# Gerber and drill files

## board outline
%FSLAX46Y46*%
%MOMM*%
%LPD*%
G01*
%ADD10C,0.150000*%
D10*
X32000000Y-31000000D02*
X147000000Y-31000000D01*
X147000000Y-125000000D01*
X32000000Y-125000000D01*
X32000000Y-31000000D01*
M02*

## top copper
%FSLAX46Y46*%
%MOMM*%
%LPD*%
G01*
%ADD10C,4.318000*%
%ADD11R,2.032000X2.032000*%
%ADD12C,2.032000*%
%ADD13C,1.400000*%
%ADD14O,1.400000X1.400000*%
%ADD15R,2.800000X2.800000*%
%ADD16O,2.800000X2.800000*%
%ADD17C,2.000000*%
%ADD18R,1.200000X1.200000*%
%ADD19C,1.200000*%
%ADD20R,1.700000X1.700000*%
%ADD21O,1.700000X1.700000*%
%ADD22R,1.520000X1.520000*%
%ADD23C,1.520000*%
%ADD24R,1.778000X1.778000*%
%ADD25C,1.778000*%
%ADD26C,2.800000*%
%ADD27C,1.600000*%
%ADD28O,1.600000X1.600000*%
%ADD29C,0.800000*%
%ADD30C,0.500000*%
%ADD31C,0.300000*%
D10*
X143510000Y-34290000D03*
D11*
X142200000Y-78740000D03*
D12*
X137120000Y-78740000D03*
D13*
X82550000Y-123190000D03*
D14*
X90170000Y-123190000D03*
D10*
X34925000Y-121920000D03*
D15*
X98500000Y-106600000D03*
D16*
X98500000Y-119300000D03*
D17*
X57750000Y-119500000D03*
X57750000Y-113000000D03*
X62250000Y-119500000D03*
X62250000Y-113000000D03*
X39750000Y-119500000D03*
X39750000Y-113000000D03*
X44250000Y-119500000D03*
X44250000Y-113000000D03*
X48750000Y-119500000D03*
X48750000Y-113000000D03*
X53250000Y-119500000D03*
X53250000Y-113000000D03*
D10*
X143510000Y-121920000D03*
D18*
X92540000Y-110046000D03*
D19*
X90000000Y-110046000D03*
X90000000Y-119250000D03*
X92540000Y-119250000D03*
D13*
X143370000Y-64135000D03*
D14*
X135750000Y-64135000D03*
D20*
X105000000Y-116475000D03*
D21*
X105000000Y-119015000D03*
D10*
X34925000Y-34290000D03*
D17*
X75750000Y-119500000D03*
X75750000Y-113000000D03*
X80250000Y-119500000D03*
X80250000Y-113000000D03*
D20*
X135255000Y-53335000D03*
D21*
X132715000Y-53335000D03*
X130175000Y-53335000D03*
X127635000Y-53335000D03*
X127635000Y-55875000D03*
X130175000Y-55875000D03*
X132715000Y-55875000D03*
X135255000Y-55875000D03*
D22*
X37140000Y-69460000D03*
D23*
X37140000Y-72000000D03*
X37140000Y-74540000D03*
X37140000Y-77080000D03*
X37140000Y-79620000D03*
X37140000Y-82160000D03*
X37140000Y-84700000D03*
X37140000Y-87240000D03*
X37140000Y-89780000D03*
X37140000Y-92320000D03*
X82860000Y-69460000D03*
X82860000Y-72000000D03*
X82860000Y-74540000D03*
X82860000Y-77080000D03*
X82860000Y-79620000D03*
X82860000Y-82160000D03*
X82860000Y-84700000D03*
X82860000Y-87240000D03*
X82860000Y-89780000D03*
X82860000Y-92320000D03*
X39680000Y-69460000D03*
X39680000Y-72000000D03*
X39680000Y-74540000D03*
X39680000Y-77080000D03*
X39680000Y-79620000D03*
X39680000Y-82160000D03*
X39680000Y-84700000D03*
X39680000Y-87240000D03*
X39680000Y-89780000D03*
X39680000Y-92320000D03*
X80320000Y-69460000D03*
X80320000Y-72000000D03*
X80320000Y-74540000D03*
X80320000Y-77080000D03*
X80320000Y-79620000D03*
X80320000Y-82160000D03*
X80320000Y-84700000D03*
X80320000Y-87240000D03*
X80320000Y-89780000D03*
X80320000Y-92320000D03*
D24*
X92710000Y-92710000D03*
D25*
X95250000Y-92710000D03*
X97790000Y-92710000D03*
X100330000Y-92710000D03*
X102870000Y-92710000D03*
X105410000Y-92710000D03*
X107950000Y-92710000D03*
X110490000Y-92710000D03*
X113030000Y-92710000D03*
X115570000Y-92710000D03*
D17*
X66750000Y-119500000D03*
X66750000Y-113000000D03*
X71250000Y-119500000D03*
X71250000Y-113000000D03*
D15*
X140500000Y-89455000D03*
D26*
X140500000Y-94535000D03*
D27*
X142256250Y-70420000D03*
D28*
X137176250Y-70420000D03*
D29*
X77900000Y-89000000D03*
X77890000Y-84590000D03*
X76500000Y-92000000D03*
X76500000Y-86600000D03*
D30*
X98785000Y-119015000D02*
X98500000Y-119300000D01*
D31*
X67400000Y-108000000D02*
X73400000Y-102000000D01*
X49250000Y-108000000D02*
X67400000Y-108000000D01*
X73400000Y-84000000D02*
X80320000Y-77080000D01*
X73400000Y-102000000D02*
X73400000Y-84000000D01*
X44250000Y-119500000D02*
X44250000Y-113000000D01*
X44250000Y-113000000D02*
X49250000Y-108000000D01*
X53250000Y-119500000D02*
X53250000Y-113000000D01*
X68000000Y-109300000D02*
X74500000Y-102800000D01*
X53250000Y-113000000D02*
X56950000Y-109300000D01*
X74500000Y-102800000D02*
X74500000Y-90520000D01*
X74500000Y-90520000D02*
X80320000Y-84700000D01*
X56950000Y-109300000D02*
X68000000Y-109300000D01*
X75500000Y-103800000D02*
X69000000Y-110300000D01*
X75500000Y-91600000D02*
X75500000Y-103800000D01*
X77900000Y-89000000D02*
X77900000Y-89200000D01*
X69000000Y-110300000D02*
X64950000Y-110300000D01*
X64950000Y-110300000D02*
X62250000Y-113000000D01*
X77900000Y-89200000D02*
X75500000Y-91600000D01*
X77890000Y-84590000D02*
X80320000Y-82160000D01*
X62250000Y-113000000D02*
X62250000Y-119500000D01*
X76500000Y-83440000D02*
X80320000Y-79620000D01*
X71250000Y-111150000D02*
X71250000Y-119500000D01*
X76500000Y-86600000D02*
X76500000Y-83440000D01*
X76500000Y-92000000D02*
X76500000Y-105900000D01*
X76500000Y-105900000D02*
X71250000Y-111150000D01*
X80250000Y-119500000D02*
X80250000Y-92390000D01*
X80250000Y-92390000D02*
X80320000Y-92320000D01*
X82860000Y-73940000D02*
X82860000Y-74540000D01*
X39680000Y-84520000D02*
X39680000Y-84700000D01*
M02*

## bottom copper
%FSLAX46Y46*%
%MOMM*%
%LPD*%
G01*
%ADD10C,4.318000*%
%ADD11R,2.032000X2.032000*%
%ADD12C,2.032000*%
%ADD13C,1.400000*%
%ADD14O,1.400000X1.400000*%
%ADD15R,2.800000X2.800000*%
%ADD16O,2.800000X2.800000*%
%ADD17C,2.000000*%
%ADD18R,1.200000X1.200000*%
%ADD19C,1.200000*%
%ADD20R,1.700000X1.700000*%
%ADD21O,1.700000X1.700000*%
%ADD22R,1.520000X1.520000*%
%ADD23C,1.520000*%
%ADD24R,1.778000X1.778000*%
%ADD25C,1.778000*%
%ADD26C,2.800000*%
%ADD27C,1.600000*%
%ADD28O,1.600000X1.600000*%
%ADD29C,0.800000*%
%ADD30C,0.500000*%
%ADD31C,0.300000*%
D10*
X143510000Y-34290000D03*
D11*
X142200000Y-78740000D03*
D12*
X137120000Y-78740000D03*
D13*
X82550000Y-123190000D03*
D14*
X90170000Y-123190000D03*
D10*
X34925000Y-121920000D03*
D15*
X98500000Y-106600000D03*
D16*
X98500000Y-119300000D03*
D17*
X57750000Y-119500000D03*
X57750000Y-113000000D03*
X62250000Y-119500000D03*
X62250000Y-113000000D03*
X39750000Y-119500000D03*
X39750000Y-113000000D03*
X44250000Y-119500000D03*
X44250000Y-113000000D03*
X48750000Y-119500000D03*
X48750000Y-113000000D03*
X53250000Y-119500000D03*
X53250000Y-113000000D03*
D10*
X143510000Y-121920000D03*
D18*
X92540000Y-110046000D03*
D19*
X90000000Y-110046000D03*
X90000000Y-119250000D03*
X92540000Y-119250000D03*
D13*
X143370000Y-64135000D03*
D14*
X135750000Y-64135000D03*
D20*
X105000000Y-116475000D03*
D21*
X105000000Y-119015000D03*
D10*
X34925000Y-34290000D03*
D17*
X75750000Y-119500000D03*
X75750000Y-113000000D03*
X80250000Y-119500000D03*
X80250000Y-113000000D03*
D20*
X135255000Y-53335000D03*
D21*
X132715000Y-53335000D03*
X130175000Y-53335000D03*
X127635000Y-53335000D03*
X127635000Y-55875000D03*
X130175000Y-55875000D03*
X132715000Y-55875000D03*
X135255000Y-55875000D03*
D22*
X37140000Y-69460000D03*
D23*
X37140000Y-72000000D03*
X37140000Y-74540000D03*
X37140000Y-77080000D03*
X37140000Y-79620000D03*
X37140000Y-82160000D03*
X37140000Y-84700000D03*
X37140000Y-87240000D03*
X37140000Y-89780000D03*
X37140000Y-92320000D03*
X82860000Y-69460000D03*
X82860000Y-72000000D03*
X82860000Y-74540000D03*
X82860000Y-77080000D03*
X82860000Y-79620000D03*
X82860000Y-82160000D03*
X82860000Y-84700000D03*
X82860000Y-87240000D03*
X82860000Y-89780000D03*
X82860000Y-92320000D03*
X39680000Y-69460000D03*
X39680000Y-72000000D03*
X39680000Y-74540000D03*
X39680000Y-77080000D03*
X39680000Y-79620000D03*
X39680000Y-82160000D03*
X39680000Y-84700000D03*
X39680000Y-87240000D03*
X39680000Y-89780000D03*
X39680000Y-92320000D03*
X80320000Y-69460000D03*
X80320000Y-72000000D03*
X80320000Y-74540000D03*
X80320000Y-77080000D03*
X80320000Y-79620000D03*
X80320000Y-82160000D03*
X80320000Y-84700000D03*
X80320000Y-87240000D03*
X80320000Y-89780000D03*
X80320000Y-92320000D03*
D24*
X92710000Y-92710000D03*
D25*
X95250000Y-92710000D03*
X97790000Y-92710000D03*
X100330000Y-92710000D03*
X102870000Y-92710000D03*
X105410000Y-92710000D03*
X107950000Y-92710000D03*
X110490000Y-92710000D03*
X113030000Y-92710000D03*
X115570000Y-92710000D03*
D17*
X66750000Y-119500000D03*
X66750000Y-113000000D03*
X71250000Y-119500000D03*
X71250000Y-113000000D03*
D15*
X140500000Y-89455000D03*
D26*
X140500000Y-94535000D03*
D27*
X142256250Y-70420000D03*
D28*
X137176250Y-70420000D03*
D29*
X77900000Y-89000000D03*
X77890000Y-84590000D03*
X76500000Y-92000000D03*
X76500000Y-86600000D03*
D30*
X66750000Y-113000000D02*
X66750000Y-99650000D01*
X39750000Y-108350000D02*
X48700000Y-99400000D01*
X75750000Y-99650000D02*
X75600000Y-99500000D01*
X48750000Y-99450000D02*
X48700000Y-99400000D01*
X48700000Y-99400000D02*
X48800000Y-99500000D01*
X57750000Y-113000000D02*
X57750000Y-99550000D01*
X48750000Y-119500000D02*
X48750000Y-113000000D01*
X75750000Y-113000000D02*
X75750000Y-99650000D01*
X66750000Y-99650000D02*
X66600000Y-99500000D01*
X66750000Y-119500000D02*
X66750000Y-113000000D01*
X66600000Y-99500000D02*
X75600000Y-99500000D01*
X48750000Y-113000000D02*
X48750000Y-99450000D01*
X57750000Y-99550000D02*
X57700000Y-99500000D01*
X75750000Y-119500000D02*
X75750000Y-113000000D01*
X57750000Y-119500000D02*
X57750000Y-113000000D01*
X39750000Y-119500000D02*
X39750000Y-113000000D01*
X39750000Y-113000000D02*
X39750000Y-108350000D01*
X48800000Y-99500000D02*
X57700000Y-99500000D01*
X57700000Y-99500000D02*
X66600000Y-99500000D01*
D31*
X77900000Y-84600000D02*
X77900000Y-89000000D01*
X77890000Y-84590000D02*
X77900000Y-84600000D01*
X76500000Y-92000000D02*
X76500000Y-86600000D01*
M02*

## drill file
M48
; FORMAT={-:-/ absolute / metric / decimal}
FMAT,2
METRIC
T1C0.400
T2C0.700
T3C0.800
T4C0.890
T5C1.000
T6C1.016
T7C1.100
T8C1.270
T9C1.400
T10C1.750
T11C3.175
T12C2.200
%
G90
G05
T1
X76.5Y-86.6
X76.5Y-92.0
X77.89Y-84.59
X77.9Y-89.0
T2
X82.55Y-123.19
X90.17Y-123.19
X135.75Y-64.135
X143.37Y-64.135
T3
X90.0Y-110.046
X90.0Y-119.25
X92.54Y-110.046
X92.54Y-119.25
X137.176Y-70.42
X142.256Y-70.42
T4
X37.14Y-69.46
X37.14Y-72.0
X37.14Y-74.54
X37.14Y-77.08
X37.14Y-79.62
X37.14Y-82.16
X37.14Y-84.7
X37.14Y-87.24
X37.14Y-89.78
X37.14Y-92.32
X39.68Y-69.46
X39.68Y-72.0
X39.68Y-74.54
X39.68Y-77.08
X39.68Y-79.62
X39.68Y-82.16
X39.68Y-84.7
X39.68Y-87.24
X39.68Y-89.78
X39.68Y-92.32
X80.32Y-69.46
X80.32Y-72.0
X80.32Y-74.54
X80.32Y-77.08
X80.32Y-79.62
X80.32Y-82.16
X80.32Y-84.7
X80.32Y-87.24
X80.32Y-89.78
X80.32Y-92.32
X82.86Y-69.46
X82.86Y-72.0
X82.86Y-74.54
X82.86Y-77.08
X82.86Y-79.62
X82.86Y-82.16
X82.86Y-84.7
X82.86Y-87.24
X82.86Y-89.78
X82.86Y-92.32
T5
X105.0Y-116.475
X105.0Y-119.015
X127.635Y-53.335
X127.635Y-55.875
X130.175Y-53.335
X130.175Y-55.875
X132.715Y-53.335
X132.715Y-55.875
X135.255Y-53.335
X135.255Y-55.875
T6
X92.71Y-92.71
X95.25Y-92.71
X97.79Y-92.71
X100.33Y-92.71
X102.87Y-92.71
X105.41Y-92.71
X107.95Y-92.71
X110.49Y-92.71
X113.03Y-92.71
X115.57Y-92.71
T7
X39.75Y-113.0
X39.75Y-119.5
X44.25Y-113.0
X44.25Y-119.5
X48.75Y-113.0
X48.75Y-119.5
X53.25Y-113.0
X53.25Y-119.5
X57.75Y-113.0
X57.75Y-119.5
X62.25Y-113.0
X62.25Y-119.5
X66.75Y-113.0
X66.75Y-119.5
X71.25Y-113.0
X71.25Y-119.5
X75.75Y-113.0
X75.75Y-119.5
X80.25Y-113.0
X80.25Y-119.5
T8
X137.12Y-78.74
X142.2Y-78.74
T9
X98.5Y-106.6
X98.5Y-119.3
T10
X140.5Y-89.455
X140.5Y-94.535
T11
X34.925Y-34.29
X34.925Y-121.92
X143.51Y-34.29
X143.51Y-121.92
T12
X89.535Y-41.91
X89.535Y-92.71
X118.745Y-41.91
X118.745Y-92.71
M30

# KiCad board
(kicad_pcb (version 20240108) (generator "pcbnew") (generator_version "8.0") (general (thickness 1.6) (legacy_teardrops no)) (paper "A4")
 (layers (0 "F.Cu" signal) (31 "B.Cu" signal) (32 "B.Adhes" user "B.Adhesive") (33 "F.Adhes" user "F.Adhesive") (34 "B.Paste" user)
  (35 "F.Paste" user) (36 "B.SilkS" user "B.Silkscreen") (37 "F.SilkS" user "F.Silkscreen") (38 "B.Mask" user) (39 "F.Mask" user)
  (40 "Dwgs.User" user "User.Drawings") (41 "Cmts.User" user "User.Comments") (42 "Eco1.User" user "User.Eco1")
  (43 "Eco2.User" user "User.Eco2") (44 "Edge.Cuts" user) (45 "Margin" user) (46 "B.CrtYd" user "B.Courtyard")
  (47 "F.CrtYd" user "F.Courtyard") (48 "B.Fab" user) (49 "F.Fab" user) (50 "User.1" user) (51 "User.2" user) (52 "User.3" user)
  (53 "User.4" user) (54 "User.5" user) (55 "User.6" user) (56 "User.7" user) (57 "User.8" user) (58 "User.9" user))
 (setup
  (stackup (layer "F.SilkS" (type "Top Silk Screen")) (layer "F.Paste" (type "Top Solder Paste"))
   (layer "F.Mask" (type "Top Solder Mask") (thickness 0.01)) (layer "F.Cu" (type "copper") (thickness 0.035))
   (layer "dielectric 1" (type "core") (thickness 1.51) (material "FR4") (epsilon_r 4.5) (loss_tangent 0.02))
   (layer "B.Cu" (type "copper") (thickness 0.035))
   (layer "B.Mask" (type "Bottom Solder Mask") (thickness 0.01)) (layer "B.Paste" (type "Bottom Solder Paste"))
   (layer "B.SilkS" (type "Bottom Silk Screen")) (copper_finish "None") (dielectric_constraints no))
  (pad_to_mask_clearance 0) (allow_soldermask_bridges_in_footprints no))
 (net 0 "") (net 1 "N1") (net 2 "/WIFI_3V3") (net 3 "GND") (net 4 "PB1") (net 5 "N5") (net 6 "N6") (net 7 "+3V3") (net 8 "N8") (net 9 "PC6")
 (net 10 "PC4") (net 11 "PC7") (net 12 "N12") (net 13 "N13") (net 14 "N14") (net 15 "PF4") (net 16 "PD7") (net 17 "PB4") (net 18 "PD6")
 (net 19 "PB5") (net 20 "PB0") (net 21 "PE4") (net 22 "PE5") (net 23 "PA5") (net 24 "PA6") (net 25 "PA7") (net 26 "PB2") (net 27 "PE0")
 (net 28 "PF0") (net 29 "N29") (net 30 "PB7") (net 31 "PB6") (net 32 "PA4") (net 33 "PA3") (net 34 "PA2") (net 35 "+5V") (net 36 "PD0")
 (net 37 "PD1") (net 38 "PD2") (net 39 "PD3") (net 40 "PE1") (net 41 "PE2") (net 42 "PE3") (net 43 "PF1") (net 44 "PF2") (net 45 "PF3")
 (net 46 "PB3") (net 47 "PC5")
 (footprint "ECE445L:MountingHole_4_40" (layer "F.Cu") (at 143.51 34.29)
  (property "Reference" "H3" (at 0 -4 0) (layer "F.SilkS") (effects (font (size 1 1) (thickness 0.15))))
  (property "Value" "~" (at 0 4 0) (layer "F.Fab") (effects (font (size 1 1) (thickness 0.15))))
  (pad "1" thru_hole circle (at 0 0) (size 4.318 4.318) (drill 3.175) (layers "*.Cu" "*.Mask") (remove_unused_layers no) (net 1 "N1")))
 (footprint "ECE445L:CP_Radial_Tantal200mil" (layer "F.Cu") (at 142.2 78.74 180)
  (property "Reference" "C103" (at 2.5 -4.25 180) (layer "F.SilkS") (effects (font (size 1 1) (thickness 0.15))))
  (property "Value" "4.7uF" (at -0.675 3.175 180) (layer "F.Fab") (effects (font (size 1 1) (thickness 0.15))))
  (pad "1" thru_hole rect (at 0 0 180) (size 2.032 2.032) (drill 1.27) (layers "*.Cu" "*.Mask") (remove_unused_layers no)
   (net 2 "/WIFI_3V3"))
  (pad "2" thru_hole circle (at 5.08 0 180) (size 2.032 2.032) (drill 1.27) (layers "*.Cu" "*.Mask") (remove_unused_layers no) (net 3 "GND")))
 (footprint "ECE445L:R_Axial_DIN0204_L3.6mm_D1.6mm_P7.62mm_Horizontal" (layer "F.Cu") (at 82.55 123.19)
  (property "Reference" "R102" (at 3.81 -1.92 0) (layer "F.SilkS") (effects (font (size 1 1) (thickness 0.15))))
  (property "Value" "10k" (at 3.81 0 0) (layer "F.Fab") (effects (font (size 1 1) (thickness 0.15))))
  (pad "1" thru_hole circle (at 0 0) (size 1.4 1.4) (drill 0.7) (layers "*.Cu" "*.Mask") (remove_unused_layers no) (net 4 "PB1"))
  (pad "2" thru_hole oval (at 7.62 0) (size 1.4 1.4) (drill 0.7) (layers "*.Cu" "*.Mask") (remove_unused_layers no) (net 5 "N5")))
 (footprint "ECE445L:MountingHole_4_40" (layer "F.Cu") (at 34.925 121.92)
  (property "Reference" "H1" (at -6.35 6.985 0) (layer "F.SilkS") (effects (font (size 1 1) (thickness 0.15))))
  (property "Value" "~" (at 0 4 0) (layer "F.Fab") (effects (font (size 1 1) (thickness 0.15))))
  (pad "1" thru_hole circle (at 0 0) (size 4.318 4.318) (drill 3.175) (layers "*.Cu" "*.Mask") (remove_unused_layers no) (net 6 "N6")))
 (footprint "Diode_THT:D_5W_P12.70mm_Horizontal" (layer "F.Cu") (at 98.5 106.6 -90)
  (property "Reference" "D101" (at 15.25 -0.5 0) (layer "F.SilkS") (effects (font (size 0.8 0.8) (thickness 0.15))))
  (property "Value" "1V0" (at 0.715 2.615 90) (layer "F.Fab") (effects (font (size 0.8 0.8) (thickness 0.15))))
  (pad "1" thru_hole rect (at 0 0 270) (size 2.8 2.8) (drill 1.4) (layers "*.Cu" "*.Mask") (remove_unused_layers no) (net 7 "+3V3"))
  (pad "2" thru_hole oval (at 12.7 0 270) (size 2.8 2.8) (drill 1.4) (layers "*.Cu" "*.Mask") (remove_unused_layers no) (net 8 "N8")))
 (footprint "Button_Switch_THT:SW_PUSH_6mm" (layer "F.Cu") (at 57.75 119.5 90)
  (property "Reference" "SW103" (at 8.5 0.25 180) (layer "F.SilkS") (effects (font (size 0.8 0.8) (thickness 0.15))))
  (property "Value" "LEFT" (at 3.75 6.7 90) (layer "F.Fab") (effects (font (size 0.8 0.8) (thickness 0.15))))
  (pad "1" thru_hole circle (at 0 0 180) (size 2 2) (drill 1.1) (layers "*.Cu" "*.Mask") (remove_unused_layers no) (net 3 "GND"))
  (pad "1" thru_hole circle (at 6.5 0 180) (size 2 2) (drill 1.1) (layers "*.Cu" "*.Mask") (remove_unused_layers no) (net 3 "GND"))
  (pad "2" thru_hole circle (at 0 4.5 180) (size 2 2) (drill 1.1) (layers "*.Cu" "*.Mask") (remove_unused_layers no) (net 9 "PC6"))
  (pad "2" thru_hole circle (at 6.5 4.5 180) (size 2 2) (drill 1.1) (layers "*.Cu" "*.Mask") (remove_unused_layers no) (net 9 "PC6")))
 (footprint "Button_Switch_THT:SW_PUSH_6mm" (layer "F.Cu") (at 39.75 119.5 90)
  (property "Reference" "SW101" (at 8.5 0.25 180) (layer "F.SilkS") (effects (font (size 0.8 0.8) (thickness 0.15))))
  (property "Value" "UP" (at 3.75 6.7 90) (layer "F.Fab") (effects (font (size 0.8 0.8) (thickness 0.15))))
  (pad "1" thru_hole circle (at 0 0 180) (size 2 2) (drill 1.1) (layers "*.Cu" "*.Mask") (remove_unused_layers no) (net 3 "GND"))
  (pad "1" thru_hole circle (at 6.5 0 180) (size 2 2) (drill 1.1) (layers "*.Cu" "*.Mask") (remove_unused_layers no) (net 3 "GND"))
  (pad "2" thru_hole circle (at 0 4.5 180) (size 2 2) (drill 1.1) (layers "*.Cu" "*.Mask") (remove_unused_layers no) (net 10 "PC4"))
  (pad "2" thru_hole circle (at 6.5 4.5 180) (size 2 2) (drill 1.1) (layers "*.Cu" "*.Mask") (remove_unused_layers no) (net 10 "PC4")))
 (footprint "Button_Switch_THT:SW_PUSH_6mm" (layer "F.Cu") (at 48.75 119.5 90)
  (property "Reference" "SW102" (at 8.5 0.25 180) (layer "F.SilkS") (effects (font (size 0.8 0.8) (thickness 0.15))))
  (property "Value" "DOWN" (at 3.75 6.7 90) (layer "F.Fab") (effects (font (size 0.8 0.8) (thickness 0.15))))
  (pad "1" thru_hole circle (at 0 0 180) (size 2 2) (drill 1.1) (layers "*.Cu" "*.Mask") (remove_unused_layers no) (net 3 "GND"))
  (pad "1" thru_hole circle (at 6.5 0 180) (size 2 2) (drill 1.1) (layers "*.Cu" "*.Mask") (remove_unused_layers no) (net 3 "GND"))
  (pad "2" thru_hole circle (at 0 4.5 180) (size 2 2) (drill 1.1) (layers "*.Cu" "*.Mask") (remove_unused_layers no) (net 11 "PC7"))
  (pad "2" thru_hole circle (at 6.5 4.5 180) (size 2 2) (drill 1.1) (layers "*.Cu" "*.Mask") (remove_unused_layers no) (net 11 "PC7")))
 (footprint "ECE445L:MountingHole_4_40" (layer "F.Cu") (at 143.51 121.92)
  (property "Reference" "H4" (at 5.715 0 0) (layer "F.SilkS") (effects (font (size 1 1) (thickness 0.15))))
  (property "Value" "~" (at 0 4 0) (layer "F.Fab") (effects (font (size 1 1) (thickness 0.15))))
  (pad "1" thru_hole circle (at 0 0) (size 4.318 4.318) (drill 3.175) (layers "*.Cu" "*.Mask") (remove_unused_layers no) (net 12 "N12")))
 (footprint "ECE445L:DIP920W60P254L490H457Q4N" (layer "F.Cu") (at 91.27 114.648 -90)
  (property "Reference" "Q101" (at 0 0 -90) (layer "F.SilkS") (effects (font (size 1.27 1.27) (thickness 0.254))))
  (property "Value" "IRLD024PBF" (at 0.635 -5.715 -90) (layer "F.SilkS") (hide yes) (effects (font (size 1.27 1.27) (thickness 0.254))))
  (pad "1" thru_hole rect (at -4.602 -1.27 270) (size 1.2 1.2) (drill 0.8) (layers "*.Cu" "*.Mask") (remove_unused_layers no) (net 8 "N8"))
  (pad "2" thru_hole circle (at -4.602 1.27 270) (size 1.2 1.2) (drill 0.8) (layers "*.Cu" "*.Mask") (remove_unused_layers no) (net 8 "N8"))
  (pad "3" thru_hole circle (at 4.602 1.27 270) (size 1.2 1.2) (drill 0.8) (layers "*.Cu" "*.Mask") (remove_unused_layers no) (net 5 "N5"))
  (pad "4" thru_hole circle (at 4.602 -1.27 270) (size 1.2 1.2) (drill 0.8) (layers "*.Cu" "*.Mask") (remove_unused_layers no) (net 3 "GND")))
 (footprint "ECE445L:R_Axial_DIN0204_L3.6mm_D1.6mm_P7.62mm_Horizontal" (layer "F.Cu") (at 143.37 64.135 180)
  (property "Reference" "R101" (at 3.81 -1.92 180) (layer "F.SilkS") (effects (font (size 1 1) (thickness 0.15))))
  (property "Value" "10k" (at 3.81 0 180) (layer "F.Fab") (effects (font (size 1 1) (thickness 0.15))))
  (pad "1" thru_hole circle (at 0 0 180) (size 1.4 1.4) (drill 0.7) (layers "*.Cu" "*.Mask") (remove_unused_layers no) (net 2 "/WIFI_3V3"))
  (pad "2" thru_hole oval (at 7.62 0 180) (size 1.4 1.4) (drill 0.7) (layers "*.Cu" "*.Mask") (remove_unused_layers no) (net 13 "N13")))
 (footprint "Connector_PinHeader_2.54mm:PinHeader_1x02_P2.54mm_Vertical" (layer "F.Cu") (at 105 116.475)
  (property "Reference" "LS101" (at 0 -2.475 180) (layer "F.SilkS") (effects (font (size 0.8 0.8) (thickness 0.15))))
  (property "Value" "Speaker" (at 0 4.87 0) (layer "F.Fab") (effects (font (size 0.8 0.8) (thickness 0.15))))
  (pad "1" thru_hole rect (at 0 0) (size 1.7 1.7) (drill 1) (layers "*.Cu" "*.Mask") (remove_unused_layers no) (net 7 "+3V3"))
  (pad "2" thru_hole oval (at 0 2.54) (size 1.7 1.7) (drill 1) (layers "*.Cu" "*.Mask") (remove_unused_layers no) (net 8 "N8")))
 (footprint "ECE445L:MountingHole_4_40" (layer "F.Cu") (at 34.925 34.29)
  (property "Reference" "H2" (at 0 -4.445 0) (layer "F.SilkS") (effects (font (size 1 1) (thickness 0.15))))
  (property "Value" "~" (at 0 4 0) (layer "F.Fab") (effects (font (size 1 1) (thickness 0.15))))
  (pad "1" thru_hole circle (at 0 0) (size 4.318 4.318) (drill 3.175) (layers "*.Cu" "*.Mask") (remove_unused_layers no) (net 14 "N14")))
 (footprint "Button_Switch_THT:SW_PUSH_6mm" (layer "F.Cu") (at 75.75 119.5 90)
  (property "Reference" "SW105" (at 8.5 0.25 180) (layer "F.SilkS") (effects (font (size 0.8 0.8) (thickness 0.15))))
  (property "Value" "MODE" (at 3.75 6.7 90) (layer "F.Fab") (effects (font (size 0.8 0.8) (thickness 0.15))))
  (pad "1" thru_hole circle (at 0 0 180) (size 2 2) (drill 1.1) (layers "*.Cu" "*.Mask") (remove_unused_layers no) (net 3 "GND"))
  (pad "1" thru_hole circle (at 6.5 0 180) (size 2 2) (drill 1.1) (layers "*.Cu" "*.Mask") (remove_unused_layers no) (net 3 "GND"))
  (pad "2" thru_hole circle (at 0 4.5 180) (size 2 2) (drill 1.1) (layers "*.Cu" "*.Mask") (remove_unused_layers no) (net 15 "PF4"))
  (pad "2" thru_hole circle (at 6.5 4.5 180) (size 2 2) (drill 1.1) (layers "*.Cu" "*.Mask") (remove_unused_layers no) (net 15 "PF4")))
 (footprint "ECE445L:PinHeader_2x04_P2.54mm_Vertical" (layer "F.Cu") (at 135.255 53.335 -90)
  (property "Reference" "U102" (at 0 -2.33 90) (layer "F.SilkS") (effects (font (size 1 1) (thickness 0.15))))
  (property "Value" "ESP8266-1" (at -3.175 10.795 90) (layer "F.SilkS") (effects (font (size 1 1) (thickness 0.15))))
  (pad "1" thru_hole rect (at 0 0 270) (size 1.7 1.7) (drill 1) (layers "*.Cu" "*.Mask") (remove_unused_layers no) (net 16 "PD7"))
  (pad "2" thru_hole oval (at 0 2.54 270) (size 1.7 1.7) (drill 1) (layers "*.Cu" "*.Mask") (remove_unused_layers no) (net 2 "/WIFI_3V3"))
  (pad "3" thru_hole oval (at 0 5.08 270) (size 1.7 1.7) (drill 1) (layers "*.Cu" "*.Mask") (remove_unused_layers no) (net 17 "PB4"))
  (pad "4" thru_hole oval (at 0 7.62 270) (size 1.7 1.7) (drill 1) (layers "*.Cu" "*.Mask") (remove_unused_layers no) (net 3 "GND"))
  (pad "5" thru_hole oval (at 2.54 7.62 270) (size 1.7 1.7) (drill 1) (layers "*.Cu" "*.Mask") (remove_unused_layers no) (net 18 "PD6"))
  (pad "6" thru_hole oval (at 2.54 5.08 270) (size 1.7 1.7) (drill 1) (layers "*.Cu" "*.Mask") (remove_unused_layers no) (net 13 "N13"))
  (pad "7" thru_hole oval (at 2.54 2.54 270) (size 1.7 1.7) (drill 1) (layers "*.Cu" "*.Mask") (remove_unused_layers no) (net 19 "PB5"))
  (pad "8" thru_hole oval (at 2.54 0 270) (size 1.7 1.7) (drill 1) (layers "*.Cu" "*.Mask") (remove_unused_layers no) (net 2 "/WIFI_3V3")))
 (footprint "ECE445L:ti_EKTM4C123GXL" (layer "F.Cu") (at 60 72)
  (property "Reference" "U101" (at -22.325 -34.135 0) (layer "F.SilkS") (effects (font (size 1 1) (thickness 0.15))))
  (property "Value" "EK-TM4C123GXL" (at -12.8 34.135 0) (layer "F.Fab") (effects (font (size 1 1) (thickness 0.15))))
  (pad "J1_1" thru_hole rect (at -22.86 -2.54) (size 1.52 1.52) (drill 0.89) (layers "*.Cu" "*.Mask") (remove_unused_layers no)
   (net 7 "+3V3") (solder_mask_margin 0.102))
  (pad "J1_2" thru_hole circle (at -22.86 0) (size 1.52 1.52) (drill 0.89) (layers "*.Cu" "*.Mask") (remove_unused_layers no) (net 19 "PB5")
   (solder_mask_margin 0.102))
  (pad "J1_3" thru_hole circle (at -22.86 2.54) (size 1.52 1.52) (drill 0.89) (layers "*.Cu" "*.Mask") (remove_unused_layers no)
   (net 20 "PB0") (solder_mask_margin 0.102))
  (pad "J1_4" thru_hole circle (at -22.86 5.08) (size 1.52 1.52) (drill 0.89) (layers "*.Cu" "*.Mask") (remove_unused_layers no)
   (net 4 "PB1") (solder_mask_margin 0.102))
  (pad "J1_5" thru_hole circle (at -22.86 7.62) (size 1.52 1.52) (drill 0.89) (layers "*.Cu" "*.Mask") (remove_unused_layers no)
   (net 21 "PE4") (solder_mask_margin 0.102))
  (pad "J1_6" thru_hole circle (at -22.86 10.16) (size 1.52 1.52) (drill 0.89) (layers "*.Cu" "*.Mask") (remove_unused_layers no)
   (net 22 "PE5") (solder_mask_margin 0.102))
  (pad "J1_7" thru_hole circle (at -22.86 12.7) (size 1.52 1.52) (drill 0.89) (layers "*.Cu" "*.Mask") (remove_unused_layers no)
   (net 17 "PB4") (solder_mask_margin 0.102))
  (pad "J1_8" thru_hole circle (at -22.86 15.24) (size 1.52 1.52) (drill 0.89) (layers "*.Cu" "*.Mask") (remove_unused_layers no)
   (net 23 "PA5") (solder_mask_margin 0.102))
  (pad "J1_9" thru_hole circle (at -22.86 17.78) (size 1.52 1.52) (drill 0.89) (layers "*.Cu" "*.Mask") (remove_unused_layers no)
   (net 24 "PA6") (solder_mask_margin 0.102))
  (pad "J1_10" thru_hole circle (at -22.86 20.32) (size 1.52 1.52) (drill 0.89) (layers "*.Cu" "*.Mask") (remove_unused_layers no)
   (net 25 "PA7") (solder_mask_margin 0.102))
  (pad "J2_1" thru_hole circle (at 22.86 -2.54) (size 1.52 1.52) (drill 0.89) (layers "*.Cu" "*.Mask") (remove_unused_layers no)
   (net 3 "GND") (solder_mask_margin 0.102))
  (pad "J2_2" thru_hole circle (at 22.86 0) (size 1.52 1.52) (drill 0.89) (layers "*.Cu" "*.Mask") (remove_unused_layers no) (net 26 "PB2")
   (solder_mask_margin 0.102))
  (pad "J2_3" thru_hole circle (at 22.86 2.54) (size 1.52 1.52) (drill 0.89) (layers "*.Cu" "*.Mask") (remove_unused_layers no)
   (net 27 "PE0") (solder_mask_margin 0.102))
  (pad "J2_4" thru_hole circle (at 22.86 5.08) (size 1.52 1.52) (drill 0.89) (layers "*.Cu" "*.Mask") (remove_unused_layers no)
   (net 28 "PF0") (solder_mask_margin 0.102))
  (pad "J2_5" thru_hole circle (at 22.86 7.62) (size 1.52 1.52) (drill 0.89) (layers "*.Cu" "*.Mask") (remove_unused_layers no)
   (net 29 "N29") (solder_mask_margin 0.102))
  (pad "J2_6" thru_hole circle (at 22.86 10.16) (size 1.52 1.52) (drill 0.89) (layers "*.Cu" "*.Mask") (remove_unused_layers no)
   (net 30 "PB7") (solder_mask_margin 0.102))
  (pad "J2_7" thru_hole circle (at 22.86 12.7) (size 1.52 1.52) (drill 0.89) (layers "*.Cu" "*.Mask") (remove_unused_layers no)
   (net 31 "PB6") (solder_mask_margin 0.102))
  (pad "J2_8" thru_hole circle (at 22.86 15.24) (size 1.52 1.52) (drill 0.89) (layers "*.Cu" "*.Mask") (remove_unused_layers no)
   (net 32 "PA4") (solder_mask_margin 0.102))
  (pad "J2_9" thru_hole circle (at 22.86 17.78) (size 1.52 1.52) (drill 0.89) (layers "*.Cu" "*.Mask") (remove_unused_layers no)
   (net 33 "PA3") (solder_mask_margin 0.102))
  (pad "J2_10" thru_hole circle (at 22.86 20.32) (size 1.52 1.52) (drill 0.89) (layers "*.Cu" "*.Mask") (remove_unused_layers no)
   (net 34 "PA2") (solder_mask_margin 0.102))
  (pad "J3_1" thru_hole circle (at -20.32 -2.54) (size 1.52 1.52) (drill 0.89) (layers "*.Cu" "*.Mask") (remove_unused_layers no)
   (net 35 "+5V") (solder_mask_margin 0.102))
  (pad "J3_2" thru_hole circle (at -20.32 0) (size 1.52 1.52) (drill 0.89) (layers "*.Cu" "*.Mask") (remove_unused_layers no) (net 3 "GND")
   (solder_mask_margin 0.102))
  (pad "J3_3" thru_hole circle (at -20.32 2.54) (size 1.52 1.52) (drill 0.89) (layers "*.Cu" "*.Mask") (remove_unused_layers no)
   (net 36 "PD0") (solder_mask_margin 0.102))
  (pad "J3_4" thru_hole circle (at -20.32 5.08) (size 1.52 1.52) (drill 0.89) (layers "*.Cu" "*.Mask") (remove_unused_layers no)
   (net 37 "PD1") (solder_mask_margin 0.102))
  (pad "J3_5" thru_hole circle (at -20.32 7.62) (size 1.52 1.52) (drill 0.89) (layers "*.Cu" "*.Mask") (remove_unused_layers no)
   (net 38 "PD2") (solder_mask_margin 0.102))
  (pad "J3_6" thru_hole circle (at -20.32 10.16) (size 1.52 1.52) (drill 0.89) (layers "*.Cu" "*.Mask") (remove_unused_layers no)
   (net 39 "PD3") (solder_mask_margin 0.102))
  (pad "J3_7" thru_hole circle (at -20.32 12.7) (size 1.52 1.52) (drill 0.89) (layers "*.Cu" "*.Mask") (remove_unused_layers no)
   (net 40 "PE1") (solder_mask_margin 0.102))
  (pad "J3_8" thru_hole circle (at -20.32 15.24) (size 1.52 1.52) (drill 0.89) (layers "*.Cu" "*.Mask") (remove_unused_layers no)
   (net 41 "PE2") (solder_mask_margin 0.102))
  (pad "J3_9" thru_hole circle (at -20.32 17.78) (size 1.52 1.52) (drill 0.89) (layers "*.Cu" "*.Mask") (remove_unused_layers no)
   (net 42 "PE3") (solder_mask_margin 0.102))
  (pad "J3_10" thru_hole circle (at -20.32 20.32) (size 1.52 1.52) (drill 0.89) (layers "*.Cu" "*.Mask") (remove_unused_layers no)
   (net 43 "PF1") (solder_mask_margin 0.102))
  (pad "J4_1" thru_hole circle (at 20.32 -2.54) (size 1.52 1.52) (drill 0.89) (layers "*.Cu" "*.Mask") (remove_unused_layers no)
   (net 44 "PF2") (solder_mask_margin 0.102))
  (pad "J4_2" thru_hole circle (at 20.32 0) (size 1.52 1.52) (drill 0.89) (layers "*.Cu" "*.Mask") (remove_unused_layers no) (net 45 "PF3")
   (solder_mask_margin 0.102))
  (pad "J4_3" thru_hole circle (at 20.32 2.54) (size 1.52 1.52) (drill 0.89) (layers "*.Cu" "*.Mask") (remove_unused_layers no)
   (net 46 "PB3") (solder_mask_margin 0.102))
  (pad "J4_4" thru_hole circle (at 20.32 5.08) (size 1.52 1.52) (drill 0.89) (layers "*.Cu" "*.Mask") (remove_unused_layers no)
   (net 10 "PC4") (solder_mask_margin 0.102))
  (pad "J4_5" thru_hole circle (at 20.32 7.62) (size 1.52 1.52) (drill 0.89) (layers "*.Cu" "*.Mask") (remove_unused_layers no)
   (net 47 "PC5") (solder_mask_margin 0.102))
  (pad "J4_6" thru_hole circle (at 20.32 10.16) (size 1.52 1.52) (drill 0.89) (layers "*.Cu" "*.Mask") (remove_unused_layers no)
   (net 9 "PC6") (solder_mask_margin 0.102))
  (pad "J4_7" thru_hole circle (at 20.32 12.7) (size 1.52 1.52) (drill 0.89) (layers "*.Cu" "*.Mask") (remove_unused_layers no)
   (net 11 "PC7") (solder_mask_margin 0.102))
  (pad "J4_8" thru_hole circle (at 20.32 15.24) (size 1.52 1.52) (drill 0.89) (layers "*.Cu" "*.Mask") (remove_unused_layers no)
   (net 18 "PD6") (solder_mask_margin 0.102))
  (pad "J4_9" thru_hole circle (at 20.32 17.78) (size 1.52 1.52) (drill 0.89) (layers "*.Cu" "*.Mask") (remove_unused_layers no)
   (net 16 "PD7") (solder_mask_margin 0.102))
  (pad "J4_10" thru_hole circle (at 20.32 20.32) (size 1.52 1.52) (drill 0.89) (layers "*.Cu" "*.Mask") (remove_unused_layers no)
   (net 15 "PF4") (solder_mask_margin 0.102)))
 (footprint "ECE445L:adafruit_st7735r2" (layer "F.Cu") (at 104.14 67.31)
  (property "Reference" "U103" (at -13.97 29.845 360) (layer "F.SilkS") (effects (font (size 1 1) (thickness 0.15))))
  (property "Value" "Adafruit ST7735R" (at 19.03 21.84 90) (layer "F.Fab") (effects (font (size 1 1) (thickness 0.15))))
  (pad "" np_thru_hole circle (at -14.605 -25.4 90) (size 2.2 2.2) (drill 2.2) (layers "*.Cu" "*.Mask"))
  (pad "" np_thru_hole circle (at -14.605 25.4 90) (size 2.2 2.2) (drill 2.2) (layers "F&B.Cu" "*.Mask"))
  (pad "" np_thru_hole circle (at 14.605 -25.4 90) (size 2.2 2.2) (drill 2.2) (layers "F&B.Cu" "*.Mask"))
  (pad "" np_thru_hole circle (at 14.605 25.4 90) (size 2.2 2.2) (drill 2.2) (layers "F&B.Cu" "*.Mask"))
  (pad "1" thru_hole rect (at -11.43 25.4 90) (size 1.778 1.778) (drill 1.016) (layers "*.Cu" "*.Mask") (remove_unused_layers no)
   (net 3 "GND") (solder_mask_margin 0.102))
  (pad "2" thru_hole circle (at -8.89 25.4 90) (size 1.778 1.778) (drill 1.016) (layers "*.Cu" "*.Mask") (remove_unused_layers no)
   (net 7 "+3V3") (solder_mask_margin 0.102))
  (pad "3" thru_hole circle (at -6.35 25.4 90) (size 1.778 1.778) (drill 1.016) (layers "*.Cu" "*.Mask") (remove_unused_layers no)
   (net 25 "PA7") (solder_mask_margin 0.102))
  (pad "4" thru_hole circle (at -3.81 25.4 90) (size 1.778 1.778) (drill 1.016) (layers "*.Cu" "*.Mask") (remove_unused_layers no)
   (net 24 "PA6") (solder_mask_margin 0.102))
  (pad "5" thru_hole circle (at -1.27 25.4 90) (size 1.778 1.778) (drill 1.016) (layers "*.Cu" "*.Mask") (remove_unused_layers no)
   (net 20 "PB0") (solder_mask_margin 0.102))
  (pad "6" thru_hole circle (at 1.27 25.4 90) (size 1.778 1.778) (drill 1.016) (layers "*.Cu" "*.Mask") (remove_unused_layers no)
   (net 33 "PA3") (solder_mask_margin 0.102))
  (pad "7" thru_hole circle (at 3.81 25.4 90) (size 1.778 1.778) (drill 1.016) (layers "*.Cu" "*.Mask") (remove_unused_layers no)
   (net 23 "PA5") (solder_mask_margin 0.102))
  (pad "8" thru_hole circle (at 6.35 25.4 90) (size 1.778 1.778) (drill 1.016) (layers "*.Cu" "*.Mask") (remove_unused_layers no)
   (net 34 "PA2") (solder_mask_margin 0.102))
  (pad "9" thru_hole circle (at 8.89 25.4 90) (size 1.778 1.778) (drill 1.016) (layers "*.Cu" "*.Mask") (remove_unused_layers no)
   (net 32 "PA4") (solder_mask_margin 0.102))
  (pad "10" thru_hole circle (at 11.43 25.4 90) (size 1.778 1.778) (drill 1.016) (layers "*.Cu" "*.Mask") (remove_unused_layers no)
   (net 7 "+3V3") (solder_mask_margin 0.102)))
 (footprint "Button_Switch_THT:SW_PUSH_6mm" (layer "F.Cu") (at 66.75 119.5 90)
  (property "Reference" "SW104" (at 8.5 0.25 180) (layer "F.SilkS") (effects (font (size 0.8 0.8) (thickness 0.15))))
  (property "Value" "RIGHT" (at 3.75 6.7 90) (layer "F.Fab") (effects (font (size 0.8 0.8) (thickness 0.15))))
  (pad "1" thru_hole circle (at 0 0 180) (size 2 2) (drill 1.1) (layers "*.Cu" "*.Mask") (remove_unused_layers no) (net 3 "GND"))
  (pad "1" thru_hole circle (at 6.5 0 180) (size 2 2) (drill 1.1) (layers "*.Cu" "*.Mask") (remove_unused_layers no) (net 3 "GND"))
  (pad "2" thru_hole circle (at 0 4.5 180) (size 2 2) (drill 1.1) (layers "*.Cu" "*.Mask") (remove_unused_layers no) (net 47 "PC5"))
  (pad "2" thru_hole circle (at 6.5 4.5 180) (size 2 2) (drill 1.1) (layers "*.Cu" "*.Mask") (remove_unused_layers no) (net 47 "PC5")))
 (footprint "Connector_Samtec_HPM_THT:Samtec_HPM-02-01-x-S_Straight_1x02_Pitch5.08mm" (layer "F.Cu") (at 140.5 89.455)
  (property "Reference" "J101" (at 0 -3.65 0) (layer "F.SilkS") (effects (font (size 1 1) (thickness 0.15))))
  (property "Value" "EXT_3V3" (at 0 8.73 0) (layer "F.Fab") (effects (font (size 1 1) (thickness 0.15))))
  (pad "1" thru_hole rect (at 0 0) (size 2.8 2.8) (drill 1.75) (layers "*.Cu" "*.Mask") (remove_unused_layers no) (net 2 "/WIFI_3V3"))
  (pad "2" thru_hole circle (at 0 5.08) (size 2.8 2.8) (drill 1.75) (layers "*.Cu" "*.Mask") (remove_unused_layers no) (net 3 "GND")))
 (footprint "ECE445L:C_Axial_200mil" (layer "F.Cu") (at 142.25625 70.42 180)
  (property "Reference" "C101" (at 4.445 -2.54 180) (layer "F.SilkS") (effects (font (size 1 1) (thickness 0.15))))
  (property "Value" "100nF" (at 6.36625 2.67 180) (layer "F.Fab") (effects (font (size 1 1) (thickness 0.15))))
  (pad "1" thru_hole circle (at 0 0 180) (size 1.6 1.6) (drill 0.8) (layers "*.Cu" "*.Mask") (remove_unused_layers no) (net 2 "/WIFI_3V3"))
  (pad "2" thru_hole oval (at 5.08 0 180) (size 1.6 1.6) (drill 0.8) (layers "*.Cu" "*.Mask") (remove_unused_layers no) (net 3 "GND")))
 (gr_rect (start 32 31) (end 147 125) (stroke (width 0.15) (type default)) (fill none) (layer "Edge.Cuts"))
 (segment (start 66.75 113) (end 66.75 99.65) (width 0.5) (layer "B.Cu") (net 3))
 (segment (start 39.75 108.35) (end 48.7 99.4) (width 0.5) (layer "B.Cu") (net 3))
 (segment (start 75.75 99.65) (end 75.6 99.5) (width 0.5) (layer "B.Cu") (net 3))
 (segment (start 48.75 99.45) (end 48.7 99.4) (width 0.5) (layer "B.Cu") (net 3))
 (segment (start 48.7 99.4) (end 48.8 99.5) (width 0.5) (layer "B.Cu") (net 3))
 (segment (start 57.75 113) (end 57.75 99.55) (width 0.5) (layer "B.Cu") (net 3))
 (segment (start 48.75 119.5) (end 48.75 113) (width 0.5) (layer "B.Cu") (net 3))
 (segment (start 75.75 113) (end 75.75 99.65) (width 0.5) (layer "B.Cu") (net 3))
 (segment (start 66.75 99.65) (end 66.6 99.5) (width 0.5) (layer "B.Cu") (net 3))
 (segment (start 66.75 119.5) (end 66.75 113) (width 0.5) (layer "B.Cu") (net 3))
 (segment (start 66.6 99.5) (end 75.6 99.5) (width 0.5) (layer "B.Cu") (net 3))
 (segment (start 48.75 113) (end 48.75 99.45) (width 0.5) (layer "B.Cu") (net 3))
 (segment (start 57.75 99.55) (end 57.7 99.5) (width 0.5) (layer "B.Cu") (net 3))
 (segment (start 75.75 119.5) (end 75.75 113) (width 0.5) (layer "B.Cu") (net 3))
 (segment (start 57.75 119.5) (end 57.75 113) (width 0.5) (layer "B.Cu") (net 3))
 (segment (start 39.75 119.5) (end 39.75 113) (width 0.5) (layer "B.Cu") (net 3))
 (segment (start 39.75 113) (end 39.75 108.35) (width 0.5) (layer "B.Cu") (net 3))
 (segment (start 48.8 99.5) (end 57.7 99.5) (width 0.5) (layer "B.Cu") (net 3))
 (segment (start 57.7 99.5) (end 66.6 99.5) (width 0.5) (layer "B.Cu") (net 3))
 (segment (start 98.785 119.015) (end 98.5 119.3) (width 0.5) (layer "F.Cu") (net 8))
 (segment (start 67.4 108) (end 73.4 102) (width 0.3) (layer "F.Cu") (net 10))
 (segment (start 49.25 108) (end 67.4 108) (width 0.3) (layer "F.Cu") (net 10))
 (segment (start 73.4 84) (end 80.32 77.08) (width 0.3) (layer "F.Cu") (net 10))
 (segment (start 73.4 102) (end 73.4 84) (width 0.3) (layer "F.Cu") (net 10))
 (segment (start 44.25 119.5) (end 44.25 113) (width 0.3) (layer "F.Cu") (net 10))
 (segment (start 44.25 113) (end 49.25 108) (width 0.3) (layer "F.Cu") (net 10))
 (segment (start 53.25 119.5) (end 53.25 113) (width 0.3) (layer "F.Cu") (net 11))
 (segment (start 68 109.3) (end 74.5 102.8) (width 0.3) (layer "F.Cu") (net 11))
 (segment (start 53.25 113) (end 56.95 109.3) (width 0.3) (layer "F.Cu") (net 11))
 (segment (start 74.5 102.8) (end 74.5 90.52) (width 0.3) (layer "F.Cu") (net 11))
 (segment (start 74.5 90.52) (end 80.32 84.7) (width 0.3) (layer "F.Cu") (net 11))
 (segment (start 56.95 109.3) (end 68 109.3) (width 0.3) (layer "F.Cu") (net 11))
 (segment (start 75.5 103.8) (end 69 110.3) (width 0.3) (layer "F.Cu") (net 9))
 (segment (start 75.5 91.6) (end 75.5 103.8) (width 0.3) (layer "F.Cu") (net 9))
 (segment (start 77.9 89) (end 77.9 89.2) (width 0.3) (layer "F.Cu") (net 9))
 (segment (start 69 110.3) (end 64.95 110.3) (width 0.3) (layer "F.Cu") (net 9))
 (segment (start 64.95 110.3) (end 62.25 113) (width 0.3) (layer "F.Cu") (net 9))
 (segment (start 77.9 89.2) (end 75.5 91.6) (width 0.3) (layer "F.Cu") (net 9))
 (segment (start 77.89 84.59) (end 80.32 82.16) (width 0.3) (layer "F.Cu") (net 9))
 (segment (start 62.25 113) (end 62.25 119.5) (width 0.3) (layer "F.Cu") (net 9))
 (via (at 77.9 89) (size 0.8) (drill 0.4) (layers "F.Cu" "B.Cu") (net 9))
 (via (at 77.89 84.59) (size 0.8) (drill 0.4) (layers "F.Cu" "B.Cu") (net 9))
 (segment (start 77.9 84.6) (end 77.9 89) (width 0.3) (layer "B.Cu") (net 9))
 (segment (start 77.89 84.59) (end 77.9 84.6) (width 0.3) (layer "B.Cu") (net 9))
 (segment (start 76.5 83.44) (end 80.32 79.62) (width 0.3) (layer "F.Cu") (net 47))
 (segment (start 71.25 111.15) (end 71.25 119.5) (width 0.3) (layer "F.Cu") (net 47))
 (segment (start 76.5 86.6) (end 76.5 83.44) (width 0.3) (layer "F.Cu") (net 47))
 (segment (start 76.5 92) (end 76.5 105.9) (width 0.3) (layer "F.Cu") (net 47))
 (segment (start 76.5 105.9) (end 71.25 111.15) (width 0.3) (layer "F.Cu") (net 47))
 (via (at 76.5 92) (size 0.8) (drill 0.4) (layers "F.Cu" "B.Cu") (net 47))
 (via (at 76.5 86.6) (size 0.8) (drill 0.4) (layers "F.Cu" "B.Cu") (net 47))
 (segment (start 76.5 92) (end 76.5 86.6) (width 0.3) (layer "B.Cu") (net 47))
 (segment (start 80.25 119.5) (end 80.25 92.39) (width 0.3) (layer "F.Cu") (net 15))
 (segment (start 80.25 92.39) (end 80.32 92.32) (width 0.3) (layer "F.Cu") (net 15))
 (segment (start 82.86 73.94) (end 82.86 74.54) (width 0.3) (layer "F.Cu") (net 27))
 (segment (start 39.68 84.52) (end 39.68 84.7) (width 0.3) (layer "F.Cu") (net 40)))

